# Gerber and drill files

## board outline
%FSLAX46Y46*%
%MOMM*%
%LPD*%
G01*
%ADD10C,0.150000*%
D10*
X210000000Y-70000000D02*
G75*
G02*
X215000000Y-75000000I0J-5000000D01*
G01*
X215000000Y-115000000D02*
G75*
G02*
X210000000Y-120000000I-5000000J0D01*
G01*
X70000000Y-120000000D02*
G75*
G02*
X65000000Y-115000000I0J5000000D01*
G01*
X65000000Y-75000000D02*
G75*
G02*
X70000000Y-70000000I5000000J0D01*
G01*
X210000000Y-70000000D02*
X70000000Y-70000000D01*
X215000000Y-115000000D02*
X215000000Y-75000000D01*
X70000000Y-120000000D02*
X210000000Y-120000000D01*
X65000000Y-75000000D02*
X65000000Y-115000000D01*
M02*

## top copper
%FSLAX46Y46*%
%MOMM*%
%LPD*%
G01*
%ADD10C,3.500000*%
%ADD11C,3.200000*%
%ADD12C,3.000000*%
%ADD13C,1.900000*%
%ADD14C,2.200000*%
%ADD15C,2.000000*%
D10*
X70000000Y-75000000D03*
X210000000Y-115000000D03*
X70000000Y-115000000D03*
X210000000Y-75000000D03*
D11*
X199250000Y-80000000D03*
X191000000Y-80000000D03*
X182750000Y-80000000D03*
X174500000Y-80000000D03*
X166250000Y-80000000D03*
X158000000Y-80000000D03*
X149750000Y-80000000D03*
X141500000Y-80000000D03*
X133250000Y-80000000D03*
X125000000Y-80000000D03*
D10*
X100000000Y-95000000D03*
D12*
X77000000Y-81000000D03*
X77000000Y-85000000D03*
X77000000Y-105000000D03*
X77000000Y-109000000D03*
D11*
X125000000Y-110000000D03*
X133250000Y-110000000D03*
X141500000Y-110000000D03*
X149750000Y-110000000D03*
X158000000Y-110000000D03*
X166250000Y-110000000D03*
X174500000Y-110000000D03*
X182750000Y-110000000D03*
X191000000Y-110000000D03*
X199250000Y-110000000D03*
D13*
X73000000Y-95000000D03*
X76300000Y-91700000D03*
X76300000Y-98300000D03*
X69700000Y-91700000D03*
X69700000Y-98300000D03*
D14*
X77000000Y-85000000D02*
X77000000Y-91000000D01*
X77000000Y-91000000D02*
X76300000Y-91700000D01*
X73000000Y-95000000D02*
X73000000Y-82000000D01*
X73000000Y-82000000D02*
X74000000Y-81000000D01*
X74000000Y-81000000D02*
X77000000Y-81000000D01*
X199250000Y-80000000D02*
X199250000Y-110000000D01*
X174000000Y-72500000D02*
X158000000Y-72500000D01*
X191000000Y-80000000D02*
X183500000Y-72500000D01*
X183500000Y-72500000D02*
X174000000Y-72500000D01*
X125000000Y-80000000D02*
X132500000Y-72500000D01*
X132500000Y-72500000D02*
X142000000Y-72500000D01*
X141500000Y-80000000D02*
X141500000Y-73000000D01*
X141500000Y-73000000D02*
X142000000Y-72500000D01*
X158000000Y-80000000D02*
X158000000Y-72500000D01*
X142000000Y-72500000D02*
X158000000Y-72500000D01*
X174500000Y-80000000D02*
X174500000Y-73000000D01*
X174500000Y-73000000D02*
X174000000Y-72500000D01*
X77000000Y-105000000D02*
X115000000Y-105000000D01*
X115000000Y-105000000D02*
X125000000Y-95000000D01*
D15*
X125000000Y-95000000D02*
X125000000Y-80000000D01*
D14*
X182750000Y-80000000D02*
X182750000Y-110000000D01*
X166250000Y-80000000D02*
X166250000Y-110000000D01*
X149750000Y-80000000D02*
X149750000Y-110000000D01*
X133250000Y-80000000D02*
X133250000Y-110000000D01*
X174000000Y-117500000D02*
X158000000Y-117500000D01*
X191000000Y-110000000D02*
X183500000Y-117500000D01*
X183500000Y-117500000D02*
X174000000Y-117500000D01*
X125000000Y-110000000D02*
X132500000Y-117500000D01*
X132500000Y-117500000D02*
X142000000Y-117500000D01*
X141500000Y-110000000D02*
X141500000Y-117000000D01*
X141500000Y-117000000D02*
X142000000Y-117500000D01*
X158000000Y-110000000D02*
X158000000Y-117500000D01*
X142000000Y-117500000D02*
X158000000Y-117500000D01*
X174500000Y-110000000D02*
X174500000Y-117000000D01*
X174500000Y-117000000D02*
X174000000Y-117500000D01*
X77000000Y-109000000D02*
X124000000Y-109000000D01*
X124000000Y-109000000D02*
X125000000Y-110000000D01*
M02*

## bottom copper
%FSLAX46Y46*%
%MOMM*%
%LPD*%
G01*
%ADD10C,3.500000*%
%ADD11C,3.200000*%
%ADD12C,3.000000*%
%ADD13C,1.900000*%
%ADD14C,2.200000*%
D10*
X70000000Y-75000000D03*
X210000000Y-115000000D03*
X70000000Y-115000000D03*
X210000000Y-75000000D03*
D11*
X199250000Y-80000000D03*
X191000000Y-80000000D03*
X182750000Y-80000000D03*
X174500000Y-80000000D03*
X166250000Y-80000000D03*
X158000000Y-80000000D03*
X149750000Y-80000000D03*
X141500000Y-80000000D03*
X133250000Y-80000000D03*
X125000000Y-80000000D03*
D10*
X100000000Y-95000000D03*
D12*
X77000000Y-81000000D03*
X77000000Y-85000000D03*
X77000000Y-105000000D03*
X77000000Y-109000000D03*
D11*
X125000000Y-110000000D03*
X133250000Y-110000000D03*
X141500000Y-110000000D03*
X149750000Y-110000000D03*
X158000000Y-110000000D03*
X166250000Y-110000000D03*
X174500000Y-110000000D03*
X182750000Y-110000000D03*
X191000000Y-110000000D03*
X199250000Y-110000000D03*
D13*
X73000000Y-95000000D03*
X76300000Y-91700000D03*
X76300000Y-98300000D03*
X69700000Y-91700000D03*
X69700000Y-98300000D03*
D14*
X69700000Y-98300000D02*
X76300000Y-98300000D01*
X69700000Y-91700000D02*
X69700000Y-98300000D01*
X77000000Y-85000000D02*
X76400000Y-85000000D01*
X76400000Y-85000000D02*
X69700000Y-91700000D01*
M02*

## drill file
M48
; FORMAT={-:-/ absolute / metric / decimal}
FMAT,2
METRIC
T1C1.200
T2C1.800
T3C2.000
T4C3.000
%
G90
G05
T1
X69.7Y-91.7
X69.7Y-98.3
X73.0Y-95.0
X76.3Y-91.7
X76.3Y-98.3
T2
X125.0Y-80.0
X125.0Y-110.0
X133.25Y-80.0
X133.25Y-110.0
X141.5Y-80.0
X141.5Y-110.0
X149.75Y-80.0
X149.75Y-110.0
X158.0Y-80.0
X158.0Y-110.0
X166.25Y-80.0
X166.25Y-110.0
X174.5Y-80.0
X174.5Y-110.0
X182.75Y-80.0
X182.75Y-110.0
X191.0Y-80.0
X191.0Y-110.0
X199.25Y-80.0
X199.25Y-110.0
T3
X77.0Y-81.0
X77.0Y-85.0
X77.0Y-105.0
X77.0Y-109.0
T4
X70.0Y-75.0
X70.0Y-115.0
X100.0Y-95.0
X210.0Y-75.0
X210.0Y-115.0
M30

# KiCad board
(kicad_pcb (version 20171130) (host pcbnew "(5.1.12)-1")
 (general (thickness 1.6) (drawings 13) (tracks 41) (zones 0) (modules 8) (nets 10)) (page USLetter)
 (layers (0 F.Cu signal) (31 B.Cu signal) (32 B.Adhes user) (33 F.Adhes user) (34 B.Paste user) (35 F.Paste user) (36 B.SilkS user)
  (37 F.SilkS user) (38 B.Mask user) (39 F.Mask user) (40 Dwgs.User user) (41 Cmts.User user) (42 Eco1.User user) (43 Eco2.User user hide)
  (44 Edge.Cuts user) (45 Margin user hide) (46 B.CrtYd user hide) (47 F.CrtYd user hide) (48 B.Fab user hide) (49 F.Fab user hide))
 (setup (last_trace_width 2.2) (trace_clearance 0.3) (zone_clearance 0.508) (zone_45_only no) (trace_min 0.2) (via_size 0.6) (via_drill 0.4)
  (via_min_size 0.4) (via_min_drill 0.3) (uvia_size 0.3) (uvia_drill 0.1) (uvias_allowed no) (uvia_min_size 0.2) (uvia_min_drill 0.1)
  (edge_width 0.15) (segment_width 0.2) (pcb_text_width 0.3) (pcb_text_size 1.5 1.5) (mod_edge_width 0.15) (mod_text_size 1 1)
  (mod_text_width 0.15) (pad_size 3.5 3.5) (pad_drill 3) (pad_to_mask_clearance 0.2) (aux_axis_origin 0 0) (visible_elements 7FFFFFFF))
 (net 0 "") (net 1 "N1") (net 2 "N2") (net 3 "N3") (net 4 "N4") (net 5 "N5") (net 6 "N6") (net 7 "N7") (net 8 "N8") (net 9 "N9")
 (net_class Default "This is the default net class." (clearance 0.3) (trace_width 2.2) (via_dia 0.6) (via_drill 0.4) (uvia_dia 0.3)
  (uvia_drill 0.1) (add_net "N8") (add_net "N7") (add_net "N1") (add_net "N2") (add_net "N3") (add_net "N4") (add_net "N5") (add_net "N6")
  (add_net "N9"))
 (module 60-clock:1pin (layer F.Cu) (at 70 75)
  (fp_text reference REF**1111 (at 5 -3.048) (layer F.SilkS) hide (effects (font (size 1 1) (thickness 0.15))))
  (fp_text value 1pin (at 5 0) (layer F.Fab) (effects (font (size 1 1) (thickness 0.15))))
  (pad 1 thru_hole circle (at 0 0) (size 3.5 3.5) (drill 3) (layers *.Cu *.Mask)))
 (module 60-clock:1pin (layer F.Cu) (at 210 115)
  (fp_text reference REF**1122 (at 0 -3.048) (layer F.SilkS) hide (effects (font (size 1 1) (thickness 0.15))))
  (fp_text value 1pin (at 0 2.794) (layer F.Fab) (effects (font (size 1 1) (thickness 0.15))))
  (pad 1 thru_hole circle (at 0 0) (size 3.5 3.5) (drill 3) (layers *.Cu *.Mask)))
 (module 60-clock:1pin (layer F.Cu) (at 70 115)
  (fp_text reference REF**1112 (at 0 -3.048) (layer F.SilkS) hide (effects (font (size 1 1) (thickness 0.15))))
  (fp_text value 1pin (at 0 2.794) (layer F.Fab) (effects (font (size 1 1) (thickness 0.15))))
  (pad 1 thru_hole circle (at 0 0) (size 3.5 3.5) (drill 3) (layers *.Cu *.Mask)))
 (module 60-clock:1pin (layer F.Cu) (at 210 75)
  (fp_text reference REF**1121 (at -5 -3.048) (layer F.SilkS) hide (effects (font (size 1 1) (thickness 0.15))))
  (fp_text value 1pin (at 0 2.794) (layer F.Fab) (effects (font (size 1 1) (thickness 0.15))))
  (pad 1 thru_hole circle (at 0 0) (size 3.5 3.5) (drill 3) (layers *.Cu *.Mask)))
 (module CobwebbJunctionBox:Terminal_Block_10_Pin (layer F.Cu) (at 199.25 80 180)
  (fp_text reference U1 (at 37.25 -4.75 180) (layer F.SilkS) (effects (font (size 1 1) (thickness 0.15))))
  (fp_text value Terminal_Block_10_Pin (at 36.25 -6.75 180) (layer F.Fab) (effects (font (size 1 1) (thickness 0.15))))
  (pad 1 thru_hole circle (at 0 0 180) (size 3.2 3.2) (drill 1.8) (layers *.Cu *.Mask F.SilkS) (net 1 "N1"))
  (pad 2 thru_hole circle (at 8.25 0 180) (size 3.2 3.2) (drill 1.8) (layers *.Cu *.Mask F.SilkS) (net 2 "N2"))
  (pad 3 thru_hole circle (at 16.5 0 180) (size 3.2 3.2) (drill 1.8) (layers *.Cu *.Mask F.SilkS) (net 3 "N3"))
  (pad 4 thru_hole circle (at 24.75 0 180) (size 3.2 3.2) (drill 1.8) (layers *.Cu *.Mask F.SilkS) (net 2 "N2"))
  (pad 5 thru_hole circle (at 33 0 180) (size 3.2 3.2) (drill 1.8) (layers *.Cu *.Mask F.SilkS) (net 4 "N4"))
  (pad 6 thru_hole circle (at 41.25 0 180) (size 3.2 3.2) (drill 1.8) (layers *.Cu *.Mask F.SilkS) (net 2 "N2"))
  (pad 7 thru_hole circle (at 49.5 0 180) (size 3.2 3.2) (drill 1.8) (layers *.Cu *.Mask F.SilkS) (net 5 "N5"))
  (pad 8 thru_hole circle (at 57.75 0 180) (size 3.2 3.2) (drill 1.8) (layers *.Cu *.Mask F.SilkS) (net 2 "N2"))
  (pad 9 thru_hole circle (at 66 0 180) (size 3.2 3.2) (drill 1.8) (layers *.Cu *.Mask F.SilkS) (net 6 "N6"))
  (pad 10 thru_hole circle (at 74.25 0 180) (size 3.2 3.2) (drill 1.8) (layers *.Cu *.Mask F.SilkS) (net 2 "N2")))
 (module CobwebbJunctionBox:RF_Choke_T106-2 (layer F.Cu) (at 100 95)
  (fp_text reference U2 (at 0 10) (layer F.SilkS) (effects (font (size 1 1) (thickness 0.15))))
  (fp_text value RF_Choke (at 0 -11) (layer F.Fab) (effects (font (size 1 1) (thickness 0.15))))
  (pad "" thru_hole circle (at 0 0) (size 3.5 3.5) (drill 3) (layers *.Cu *.Mask F.SilkS))
  (pad 1 thru_hole circle (at -23 -14) (size 3 3) (drill 2) (layers *.Cu *.Mask F.SilkS) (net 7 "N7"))
  (pad 2 thru_hole circle (at -23 -10) (size 3 3) (drill 2) (layers *.Cu *.Mask F.SilkS) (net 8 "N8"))
  (pad 3 thru_hole circle (at -23 10) (size 3 3) (drill 2) (layers *.Cu *.Mask F.SilkS) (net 2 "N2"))
  (pad 4 thru_hole circle (at -23 14) (size 3 3) (drill 2) (layers *.Cu *.Mask F.SilkS) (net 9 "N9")))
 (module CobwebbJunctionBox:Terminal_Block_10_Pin (layer F.Cu) (at 125 110)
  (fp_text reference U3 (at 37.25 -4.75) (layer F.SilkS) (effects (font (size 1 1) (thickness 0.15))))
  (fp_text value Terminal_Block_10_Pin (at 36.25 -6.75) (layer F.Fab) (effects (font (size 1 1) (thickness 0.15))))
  (pad 1 thru_hole circle (at 0 0) (size 3.2 3.2) (drill 1.8) (layers *.Cu *.Mask F.SilkS) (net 9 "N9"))
  (pad 2 thru_hole circle (at 8.25 0) (size 3.2 3.2) (drill 1.8) (layers *.Cu *.Mask F.SilkS) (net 6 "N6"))
  (pad 3 thru_hole circle (at 16.5 0) (size 3.2 3.2) (drill 1.8) (layers *.Cu *.Mask F.SilkS) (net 9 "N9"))
  (pad 4 thru_hole circle (at 24.75 0) (size 3.2 3.2) (drill 1.8) (layers *.Cu *.Mask F.SilkS) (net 5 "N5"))
  (pad 5 thru_hole circle (at 33 0) (size 3.2 3.2) (drill 1.8) (layers *.Cu *.Mask F.SilkS) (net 9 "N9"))
  (pad 6 thru_hole circle (at 41.25 0) (size 3.2 3.2) (drill 1.8) (layers *.Cu *.Mask F.SilkS) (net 4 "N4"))
  (pad 7 thru_hole circle (at 49.5 0) (size 3.2 3.2) (drill 1.8) (layers *.Cu *.Mask F.SilkS) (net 9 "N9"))
  (pad 8 thru_hole circle (at 57.75 0) (size 3.2 3.2) (drill 1.8) (layers *.Cu *.Mask F.SilkS) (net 3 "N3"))
  (pad 9 thru_hole circle (at 66 0) (size 3.2 3.2) (drill 1.8) (layers *.Cu *.Mask F.SilkS) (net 9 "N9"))
  (pad 10 thru_hole circle (at 74.25 0) (size 3.2 3.2) (drill 1.8) (layers *.Cu *.Mask F.SilkS) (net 1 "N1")))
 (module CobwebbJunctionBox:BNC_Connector (layer F.Cu) (at 73 95 270)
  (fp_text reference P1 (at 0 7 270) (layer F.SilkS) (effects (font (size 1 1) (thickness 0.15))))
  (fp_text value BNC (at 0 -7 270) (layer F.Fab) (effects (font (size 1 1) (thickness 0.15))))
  (pad 2 thru_hole circle (at 0 0 270) (size 1.9 1.9) (drill 1.2) (layers *.Cu *.Mask F.SilkS) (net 7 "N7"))
  (pad 1 thru_hole circle (at -3.3 -3.3 270) (size 1.9 1.9) (drill 1.2) (layers *.Cu *.Mask F.SilkS) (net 8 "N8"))
  (pad 1 thru_hole circle (at 3.3 -3.3 270) (size 1.9 1.9) (drill 1.2) (layers *.Cu *.Mask F.SilkS) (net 8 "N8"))
  (pad 1 thru_hole circle (at -3.3 3.3 270) (size 1.9 1.9) (drill 1.2) (layers *.Cu *.Mask F.SilkS) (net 8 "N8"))
  (pad 1 thru_hole circle (at 3.3 3.3 270) (size 1.9 1.9) (drill 1.2) (layers *.Cu *.Mask F.SilkS) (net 8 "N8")))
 (gr_arc (start 210 75) (end 210 70) (angle 90) (layer Edge.Cuts) (width 0.15))
 (gr_arc (start 210 115) (end 215 115) (angle 90) (layer Edge.Cuts) (width 0.15))
 (gr_arc (start 70 115) (end 70 120) (angle 90) (layer Edge.Cuts) (width 0.15))
 (gr_arc (start 70 75) (end 65 75) (angle 90) (layer Edge.Cuts) (width 0.15))
 (gr_line (start 210 70) (end 70 70) (layer Edge.Cuts) (width 0.15))
 (gr_line (start 215 115) (end 215 75) (layer Edge.Cuts) (width 0.15))
 (gr_line (start 70 120) (end 210 120) (layer Edge.Cuts) (width 0.15))
 (gr_line (start 65 75) (end 65 115) (layer Edge.Cuts) (width 0.15))
 (segment (start 69.7 98.3) (end 76.3 98.3) (width 2.2) (layer B.Cu) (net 8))
 (segment (start 69.7 91.7) (end 69.7 98.3) (width 2.2) (layer B.Cu) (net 8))
 (segment (start 77 85) (end 76.4 85) (width 2.2) (layer B.Cu) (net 8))
 (segment (start 76.4 85) (end 69.7 91.7) (width 2.2) (layer B.Cu) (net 8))
 (segment (start 77 85) (end 77 91) (width 2.2) (layer F.Cu) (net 8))
 (segment (start 77 91) (end 76.3 91.7) (width 2.2) (layer F.Cu) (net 8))
 (segment (start 73 95) (end 73 82) (width 2.2) (layer F.Cu) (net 7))
 (segment (start 73 82) (end 74 81) (width 2.2) (layer F.Cu) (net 7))
 (segment (start 74 81) (end 77 81) (width 2.2) (layer F.Cu) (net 7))
 (segment (start 199.25 80) (end 199.25 110) (width 2.2) (layer F.Cu) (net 1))
 (segment (start 174 72.5) (end 158 72.5) (width 2.2) (layer F.Cu) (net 2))
 (segment (start 191 80) (end 183.5 72.5) (width 2.2) (layer F.Cu) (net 2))
 (segment (start 183.5 72.5) (end 174 72.5) (width 2.2) (layer F.Cu) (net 2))
 (segment (start 125 80) (end 132.5 72.5) (width 2.2) (layer F.Cu) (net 2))
 (segment (start 132.5 72.5) (end 142 72.5) (width 2.2) (layer F.Cu) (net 2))
 (segment (start 141.5 80) (end 141.5 73) (width 2.2) (layer F.Cu) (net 2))
 (segment (start 141.5 73) (end 142 72.5) (width 2.2) (layer F.Cu) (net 2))
 (segment (start 158 80) (end 158 72.5) (width 2.2) (layer F.Cu) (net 2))
 (segment (start 142 72.5) (end 158 72.5) (width 2.2) (layer F.Cu) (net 2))
 (segment (start 174.5 80) (end 174.5 73) (width 2.2) (layer F.Cu) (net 2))
 (segment (start 174.5 73) (end 174 72.5) (width 2.2) (layer F.Cu) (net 2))
 (segment (start 77 105) (end 115 105) (width 2.2) (layer F.Cu) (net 2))
 (segment (start 115 105) (end 125 95) (width 2.2) (layer F.Cu) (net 2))
 (segment (start 125 95) (end 125 80) (width 2) (layer F.Cu) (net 2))
 (segment (start 182.75 80) (end 182.75 110) (width 2.2) (layer F.Cu) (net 3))
 (segment (start 166.25 80) (end 166.25 110) (width 2.2) (layer F.Cu) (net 4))
 (segment (start 149.75 80) (end 149.75 110) (width 2.2) (layer F.Cu) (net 5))
 (segment (start 133.25 80) (end 133.25 110) (width 2.2) (layer F.Cu) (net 6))
 (segment (start 174 117.5) (end 158 117.5) (width 2.2) (layer F.Cu) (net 9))
 (segment (start 191 110) (end 183.5 117.5) (width 2.2) (layer F.Cu) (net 9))
 (segment (start 183.5 117.5) (end 174 117.5) (width 2.2) (layer F.Cu) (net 9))
 (segment (start 125 110) (end 132.5 117.5) (width 2.2) (layer F.Cu) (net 9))
 (segment (start 132.5 117.5) (end 142 117.5) (width 2.2) (layer F.Cu) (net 9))
 (segment (start 141.5 110) (end 141.5 117) (width 2.2) (layer F.Cu) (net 9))
 (segment (start 141.5 117) (end 142 117.5) (width 2.2) (layer F.Cu) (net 9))
 (segment (start 158 110) (end 158 117.5) (width 2.2) (layer F.Cu) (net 9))
 (segment (start 142 117.5) (end 158 117.5) (width 2.2) (layer F.Cu) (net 9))
 (segment (start 174.5 110) (end 174.5 117) (width 2.2) (layer F.Cu) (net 9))
 (segment (start 174.5 117) (end 174 117.5) (width 2.2) (layer F.Cu) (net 9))
 (segment (start 77 109) (end 124 109) (width 2.2) (layer F.Cu) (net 9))
 (segment (start 124 109) (end 125 110) (width 2.2) (layer F.Cu) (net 9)))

